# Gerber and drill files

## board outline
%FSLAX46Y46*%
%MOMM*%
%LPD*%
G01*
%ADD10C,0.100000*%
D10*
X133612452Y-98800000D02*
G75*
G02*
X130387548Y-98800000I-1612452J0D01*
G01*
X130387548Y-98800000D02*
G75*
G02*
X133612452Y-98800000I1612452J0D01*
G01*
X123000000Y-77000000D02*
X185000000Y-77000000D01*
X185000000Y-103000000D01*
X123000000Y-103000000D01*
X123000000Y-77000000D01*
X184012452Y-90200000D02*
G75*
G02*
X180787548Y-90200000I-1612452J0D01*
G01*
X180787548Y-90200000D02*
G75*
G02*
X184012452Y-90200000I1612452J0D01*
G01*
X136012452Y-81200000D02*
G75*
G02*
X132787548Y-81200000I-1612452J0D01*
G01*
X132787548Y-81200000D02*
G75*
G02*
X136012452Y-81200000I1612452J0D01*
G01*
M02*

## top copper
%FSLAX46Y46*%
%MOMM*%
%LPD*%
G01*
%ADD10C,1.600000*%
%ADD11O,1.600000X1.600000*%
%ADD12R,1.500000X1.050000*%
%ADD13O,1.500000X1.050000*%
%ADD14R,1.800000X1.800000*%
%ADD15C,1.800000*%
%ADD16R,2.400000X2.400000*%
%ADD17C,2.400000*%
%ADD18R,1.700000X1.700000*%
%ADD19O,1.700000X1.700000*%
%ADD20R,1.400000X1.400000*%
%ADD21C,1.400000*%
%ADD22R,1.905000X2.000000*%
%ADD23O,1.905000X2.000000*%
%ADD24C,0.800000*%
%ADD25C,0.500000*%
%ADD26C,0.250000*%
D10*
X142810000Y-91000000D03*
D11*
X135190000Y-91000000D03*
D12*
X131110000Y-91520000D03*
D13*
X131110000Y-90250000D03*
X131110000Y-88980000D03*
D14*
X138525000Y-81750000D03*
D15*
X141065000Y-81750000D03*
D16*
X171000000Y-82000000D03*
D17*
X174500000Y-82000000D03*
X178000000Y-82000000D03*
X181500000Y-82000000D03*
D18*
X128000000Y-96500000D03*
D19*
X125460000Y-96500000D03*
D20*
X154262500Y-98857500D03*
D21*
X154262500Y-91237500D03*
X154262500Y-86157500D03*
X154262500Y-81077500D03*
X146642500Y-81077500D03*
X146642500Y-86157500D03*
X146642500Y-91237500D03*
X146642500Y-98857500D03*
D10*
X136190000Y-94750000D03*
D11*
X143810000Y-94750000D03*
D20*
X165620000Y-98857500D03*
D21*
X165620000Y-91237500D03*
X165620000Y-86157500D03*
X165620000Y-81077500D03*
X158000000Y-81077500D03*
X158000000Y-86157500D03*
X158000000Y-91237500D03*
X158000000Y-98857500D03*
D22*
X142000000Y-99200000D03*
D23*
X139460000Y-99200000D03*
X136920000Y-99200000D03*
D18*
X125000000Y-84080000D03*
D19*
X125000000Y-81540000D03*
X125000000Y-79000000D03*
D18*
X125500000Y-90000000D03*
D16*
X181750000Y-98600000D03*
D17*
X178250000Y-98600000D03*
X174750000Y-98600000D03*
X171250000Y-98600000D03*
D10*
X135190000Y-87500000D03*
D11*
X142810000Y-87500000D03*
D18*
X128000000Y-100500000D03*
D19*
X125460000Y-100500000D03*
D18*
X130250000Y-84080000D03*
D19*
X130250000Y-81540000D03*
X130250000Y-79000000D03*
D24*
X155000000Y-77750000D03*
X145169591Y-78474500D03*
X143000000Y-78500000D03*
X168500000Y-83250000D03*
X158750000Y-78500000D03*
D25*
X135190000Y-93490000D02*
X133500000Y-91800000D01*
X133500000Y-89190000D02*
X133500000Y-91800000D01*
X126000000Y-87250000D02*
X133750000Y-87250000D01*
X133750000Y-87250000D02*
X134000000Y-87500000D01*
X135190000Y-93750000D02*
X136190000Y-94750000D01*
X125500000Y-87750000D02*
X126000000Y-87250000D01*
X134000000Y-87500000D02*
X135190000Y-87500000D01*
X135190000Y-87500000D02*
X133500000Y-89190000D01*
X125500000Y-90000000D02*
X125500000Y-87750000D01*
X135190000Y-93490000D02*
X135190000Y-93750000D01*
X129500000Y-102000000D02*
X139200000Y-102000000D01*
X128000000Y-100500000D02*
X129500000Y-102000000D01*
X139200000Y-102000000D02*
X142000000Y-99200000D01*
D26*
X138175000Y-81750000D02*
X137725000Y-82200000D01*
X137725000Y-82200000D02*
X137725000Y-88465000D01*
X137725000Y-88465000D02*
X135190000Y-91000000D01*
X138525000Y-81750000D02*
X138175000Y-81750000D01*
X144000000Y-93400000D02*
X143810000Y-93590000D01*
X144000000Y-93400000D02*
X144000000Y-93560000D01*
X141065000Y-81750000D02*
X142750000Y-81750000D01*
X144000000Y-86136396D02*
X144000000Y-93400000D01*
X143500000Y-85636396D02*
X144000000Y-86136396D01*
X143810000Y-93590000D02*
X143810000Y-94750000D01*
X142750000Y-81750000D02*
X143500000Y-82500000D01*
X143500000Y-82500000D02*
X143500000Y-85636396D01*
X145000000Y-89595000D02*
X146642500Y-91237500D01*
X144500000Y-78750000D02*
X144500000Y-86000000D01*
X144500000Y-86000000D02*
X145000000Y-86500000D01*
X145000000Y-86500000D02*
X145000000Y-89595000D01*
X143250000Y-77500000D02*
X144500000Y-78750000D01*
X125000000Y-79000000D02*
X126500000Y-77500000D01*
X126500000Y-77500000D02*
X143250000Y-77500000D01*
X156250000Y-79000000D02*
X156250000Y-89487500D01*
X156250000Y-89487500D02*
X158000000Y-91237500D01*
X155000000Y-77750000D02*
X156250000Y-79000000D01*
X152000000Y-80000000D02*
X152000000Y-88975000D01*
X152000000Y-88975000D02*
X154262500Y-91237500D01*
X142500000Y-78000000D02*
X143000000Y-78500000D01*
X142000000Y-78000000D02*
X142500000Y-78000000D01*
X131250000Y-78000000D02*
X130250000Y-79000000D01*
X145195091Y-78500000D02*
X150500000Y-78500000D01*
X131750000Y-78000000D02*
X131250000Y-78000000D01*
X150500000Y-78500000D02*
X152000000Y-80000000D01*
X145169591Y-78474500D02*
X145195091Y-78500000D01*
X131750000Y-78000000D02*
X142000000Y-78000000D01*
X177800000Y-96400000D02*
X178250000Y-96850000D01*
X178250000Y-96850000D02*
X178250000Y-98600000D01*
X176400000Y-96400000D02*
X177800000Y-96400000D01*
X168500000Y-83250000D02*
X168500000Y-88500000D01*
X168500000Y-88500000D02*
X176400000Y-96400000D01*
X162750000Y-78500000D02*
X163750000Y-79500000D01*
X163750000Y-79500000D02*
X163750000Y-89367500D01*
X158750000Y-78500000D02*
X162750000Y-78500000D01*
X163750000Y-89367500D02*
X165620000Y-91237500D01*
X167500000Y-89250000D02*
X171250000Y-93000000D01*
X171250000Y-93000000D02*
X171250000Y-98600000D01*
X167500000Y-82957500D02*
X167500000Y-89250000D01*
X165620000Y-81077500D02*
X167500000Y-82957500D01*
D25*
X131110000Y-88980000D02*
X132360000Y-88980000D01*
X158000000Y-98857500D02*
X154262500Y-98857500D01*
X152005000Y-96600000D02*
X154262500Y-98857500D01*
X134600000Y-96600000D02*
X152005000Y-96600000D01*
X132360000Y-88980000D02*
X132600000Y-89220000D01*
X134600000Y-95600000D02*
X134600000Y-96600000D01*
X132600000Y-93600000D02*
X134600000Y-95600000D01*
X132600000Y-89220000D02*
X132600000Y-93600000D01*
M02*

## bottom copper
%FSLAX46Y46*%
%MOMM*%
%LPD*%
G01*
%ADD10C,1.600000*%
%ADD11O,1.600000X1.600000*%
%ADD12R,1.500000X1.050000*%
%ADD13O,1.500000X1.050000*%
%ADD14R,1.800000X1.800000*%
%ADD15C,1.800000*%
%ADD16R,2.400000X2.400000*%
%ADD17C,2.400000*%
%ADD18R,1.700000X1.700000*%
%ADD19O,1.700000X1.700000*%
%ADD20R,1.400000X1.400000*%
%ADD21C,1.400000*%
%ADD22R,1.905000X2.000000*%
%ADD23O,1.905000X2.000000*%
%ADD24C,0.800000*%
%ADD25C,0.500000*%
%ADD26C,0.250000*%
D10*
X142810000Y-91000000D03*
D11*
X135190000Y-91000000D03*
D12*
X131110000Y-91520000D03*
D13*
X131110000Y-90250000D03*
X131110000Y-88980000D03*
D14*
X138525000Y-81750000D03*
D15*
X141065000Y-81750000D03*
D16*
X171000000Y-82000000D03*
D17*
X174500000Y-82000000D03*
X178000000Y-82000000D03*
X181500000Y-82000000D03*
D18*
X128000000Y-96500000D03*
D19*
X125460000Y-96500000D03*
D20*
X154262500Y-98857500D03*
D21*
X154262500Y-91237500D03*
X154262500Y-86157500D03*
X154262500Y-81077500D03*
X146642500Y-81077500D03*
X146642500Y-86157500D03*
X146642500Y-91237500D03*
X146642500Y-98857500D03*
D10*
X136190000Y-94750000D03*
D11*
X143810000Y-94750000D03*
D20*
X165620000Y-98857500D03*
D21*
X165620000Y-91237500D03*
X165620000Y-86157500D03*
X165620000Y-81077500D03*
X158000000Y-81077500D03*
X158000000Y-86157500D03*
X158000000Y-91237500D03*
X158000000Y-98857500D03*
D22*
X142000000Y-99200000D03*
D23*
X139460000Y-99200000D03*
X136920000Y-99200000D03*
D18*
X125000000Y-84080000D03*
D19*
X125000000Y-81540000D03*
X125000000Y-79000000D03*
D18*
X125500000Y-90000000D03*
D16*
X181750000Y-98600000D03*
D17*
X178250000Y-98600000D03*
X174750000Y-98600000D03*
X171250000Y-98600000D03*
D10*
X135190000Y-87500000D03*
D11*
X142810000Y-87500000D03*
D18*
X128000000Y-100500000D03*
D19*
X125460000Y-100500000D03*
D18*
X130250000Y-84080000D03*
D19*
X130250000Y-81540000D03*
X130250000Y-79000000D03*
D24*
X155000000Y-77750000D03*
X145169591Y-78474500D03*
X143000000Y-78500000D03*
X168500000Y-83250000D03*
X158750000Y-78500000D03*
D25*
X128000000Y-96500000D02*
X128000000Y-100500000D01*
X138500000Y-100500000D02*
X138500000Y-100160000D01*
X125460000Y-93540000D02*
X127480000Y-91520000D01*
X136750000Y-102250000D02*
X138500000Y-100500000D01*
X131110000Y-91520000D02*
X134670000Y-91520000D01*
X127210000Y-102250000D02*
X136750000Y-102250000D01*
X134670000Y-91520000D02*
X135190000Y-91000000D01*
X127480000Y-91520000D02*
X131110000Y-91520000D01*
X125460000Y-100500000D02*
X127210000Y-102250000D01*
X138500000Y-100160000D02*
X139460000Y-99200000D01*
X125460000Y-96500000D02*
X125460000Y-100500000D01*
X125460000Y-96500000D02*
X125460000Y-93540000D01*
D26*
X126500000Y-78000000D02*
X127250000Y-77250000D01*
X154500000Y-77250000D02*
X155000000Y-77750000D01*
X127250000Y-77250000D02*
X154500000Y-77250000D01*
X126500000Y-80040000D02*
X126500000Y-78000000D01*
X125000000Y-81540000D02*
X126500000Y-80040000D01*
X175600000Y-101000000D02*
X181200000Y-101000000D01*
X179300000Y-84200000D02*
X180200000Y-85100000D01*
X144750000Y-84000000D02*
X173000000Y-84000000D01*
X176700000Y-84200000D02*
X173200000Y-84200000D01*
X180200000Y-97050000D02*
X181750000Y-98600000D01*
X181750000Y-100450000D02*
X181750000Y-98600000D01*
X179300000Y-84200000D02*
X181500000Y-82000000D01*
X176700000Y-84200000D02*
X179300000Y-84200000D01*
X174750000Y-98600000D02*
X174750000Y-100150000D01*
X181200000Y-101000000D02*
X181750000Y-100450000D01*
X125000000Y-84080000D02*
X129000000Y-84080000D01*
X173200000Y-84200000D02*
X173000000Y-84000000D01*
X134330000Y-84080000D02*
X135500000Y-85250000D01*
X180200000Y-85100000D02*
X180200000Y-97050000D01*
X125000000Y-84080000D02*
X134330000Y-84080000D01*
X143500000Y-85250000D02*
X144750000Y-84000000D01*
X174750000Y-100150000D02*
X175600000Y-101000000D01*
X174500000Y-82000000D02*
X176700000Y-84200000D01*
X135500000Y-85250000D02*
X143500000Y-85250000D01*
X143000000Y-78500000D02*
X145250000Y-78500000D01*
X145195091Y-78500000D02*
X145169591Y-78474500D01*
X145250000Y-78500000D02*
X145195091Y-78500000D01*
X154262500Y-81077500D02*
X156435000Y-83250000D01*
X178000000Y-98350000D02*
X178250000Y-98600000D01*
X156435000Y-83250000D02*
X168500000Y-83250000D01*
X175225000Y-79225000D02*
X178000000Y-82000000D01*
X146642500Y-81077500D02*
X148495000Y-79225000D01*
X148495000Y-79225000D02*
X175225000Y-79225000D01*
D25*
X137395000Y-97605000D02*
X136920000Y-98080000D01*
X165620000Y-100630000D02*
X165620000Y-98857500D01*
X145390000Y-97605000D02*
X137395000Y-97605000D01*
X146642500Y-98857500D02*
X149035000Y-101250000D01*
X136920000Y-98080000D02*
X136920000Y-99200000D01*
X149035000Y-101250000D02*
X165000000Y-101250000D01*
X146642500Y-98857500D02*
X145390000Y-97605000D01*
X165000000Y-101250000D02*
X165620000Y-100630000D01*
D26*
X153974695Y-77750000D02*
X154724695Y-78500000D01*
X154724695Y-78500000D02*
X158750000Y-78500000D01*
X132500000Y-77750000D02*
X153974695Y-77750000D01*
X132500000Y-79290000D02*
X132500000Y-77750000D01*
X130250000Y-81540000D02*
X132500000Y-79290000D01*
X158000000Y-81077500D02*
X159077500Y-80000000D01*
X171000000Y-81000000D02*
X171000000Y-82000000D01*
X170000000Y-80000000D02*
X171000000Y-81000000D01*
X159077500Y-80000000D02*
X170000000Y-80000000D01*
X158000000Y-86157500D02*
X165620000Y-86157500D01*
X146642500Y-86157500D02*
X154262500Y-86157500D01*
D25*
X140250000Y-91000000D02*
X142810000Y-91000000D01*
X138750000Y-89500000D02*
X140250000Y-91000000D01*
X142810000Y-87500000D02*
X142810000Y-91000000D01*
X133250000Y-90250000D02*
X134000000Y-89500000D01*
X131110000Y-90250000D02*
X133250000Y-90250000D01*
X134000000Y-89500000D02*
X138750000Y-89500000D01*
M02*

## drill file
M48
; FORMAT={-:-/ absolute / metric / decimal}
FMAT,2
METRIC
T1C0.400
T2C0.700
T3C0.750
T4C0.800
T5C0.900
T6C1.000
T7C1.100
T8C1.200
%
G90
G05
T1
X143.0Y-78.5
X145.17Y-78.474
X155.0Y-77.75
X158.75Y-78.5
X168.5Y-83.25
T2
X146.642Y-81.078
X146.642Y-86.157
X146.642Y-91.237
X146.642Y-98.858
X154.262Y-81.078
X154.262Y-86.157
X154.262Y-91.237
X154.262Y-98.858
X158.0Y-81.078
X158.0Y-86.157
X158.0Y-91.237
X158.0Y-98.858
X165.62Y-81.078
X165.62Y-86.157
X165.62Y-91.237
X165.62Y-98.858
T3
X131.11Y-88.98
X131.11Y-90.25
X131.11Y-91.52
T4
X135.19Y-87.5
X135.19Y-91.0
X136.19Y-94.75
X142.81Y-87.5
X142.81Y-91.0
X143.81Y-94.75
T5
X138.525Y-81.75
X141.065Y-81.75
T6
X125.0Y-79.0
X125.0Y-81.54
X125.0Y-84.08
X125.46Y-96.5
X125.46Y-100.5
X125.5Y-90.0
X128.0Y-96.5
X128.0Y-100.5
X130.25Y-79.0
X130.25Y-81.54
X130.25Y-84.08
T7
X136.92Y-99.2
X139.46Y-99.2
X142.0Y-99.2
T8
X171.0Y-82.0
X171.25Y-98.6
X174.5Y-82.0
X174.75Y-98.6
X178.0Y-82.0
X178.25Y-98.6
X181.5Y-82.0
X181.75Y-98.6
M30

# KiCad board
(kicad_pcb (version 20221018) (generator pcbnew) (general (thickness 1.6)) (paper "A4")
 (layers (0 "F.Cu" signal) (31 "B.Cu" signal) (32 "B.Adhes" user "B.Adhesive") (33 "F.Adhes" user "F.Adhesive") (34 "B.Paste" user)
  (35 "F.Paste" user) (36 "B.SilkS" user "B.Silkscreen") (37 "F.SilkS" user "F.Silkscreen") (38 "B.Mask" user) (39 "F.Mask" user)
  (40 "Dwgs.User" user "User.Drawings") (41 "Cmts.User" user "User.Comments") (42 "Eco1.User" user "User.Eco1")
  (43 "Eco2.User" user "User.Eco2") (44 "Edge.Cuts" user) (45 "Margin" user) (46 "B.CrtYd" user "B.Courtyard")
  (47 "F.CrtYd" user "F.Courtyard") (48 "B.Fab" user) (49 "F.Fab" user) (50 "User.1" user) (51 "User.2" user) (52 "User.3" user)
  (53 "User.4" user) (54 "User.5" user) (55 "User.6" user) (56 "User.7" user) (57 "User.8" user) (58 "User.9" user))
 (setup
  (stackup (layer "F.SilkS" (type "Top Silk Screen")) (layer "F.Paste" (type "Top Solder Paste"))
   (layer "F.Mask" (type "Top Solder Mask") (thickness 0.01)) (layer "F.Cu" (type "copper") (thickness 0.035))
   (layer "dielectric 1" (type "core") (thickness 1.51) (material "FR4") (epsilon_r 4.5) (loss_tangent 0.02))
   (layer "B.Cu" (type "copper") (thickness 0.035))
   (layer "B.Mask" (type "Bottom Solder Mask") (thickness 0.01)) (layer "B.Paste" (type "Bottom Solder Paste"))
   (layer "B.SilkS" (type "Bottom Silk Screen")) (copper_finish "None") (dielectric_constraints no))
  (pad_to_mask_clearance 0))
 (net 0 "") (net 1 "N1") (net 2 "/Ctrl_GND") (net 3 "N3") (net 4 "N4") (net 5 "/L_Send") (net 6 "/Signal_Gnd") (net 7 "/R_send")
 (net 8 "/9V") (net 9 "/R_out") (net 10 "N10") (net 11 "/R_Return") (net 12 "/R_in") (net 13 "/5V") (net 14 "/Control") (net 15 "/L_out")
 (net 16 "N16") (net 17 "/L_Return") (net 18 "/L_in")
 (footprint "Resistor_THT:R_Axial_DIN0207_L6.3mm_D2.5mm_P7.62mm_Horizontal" (layer "F.Cu") (at 142.81 91 180)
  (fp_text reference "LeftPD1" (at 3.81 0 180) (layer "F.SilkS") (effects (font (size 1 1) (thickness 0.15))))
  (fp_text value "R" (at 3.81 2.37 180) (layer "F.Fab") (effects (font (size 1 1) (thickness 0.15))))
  (pad "1" thru_hole circle (at 0 0 180) (size 1.6 1.6) (drill 0.8) (layers "*.Cu" "*.Mask") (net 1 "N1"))
  (pad "2" thru_hole oval (at 7.62 0 180) (size 1.6 1.6) (drill 0.8) (layers "*.Cu" "*.Mask") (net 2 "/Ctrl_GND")))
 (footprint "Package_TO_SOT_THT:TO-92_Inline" (layer "F.Cu") (at 131.11 91.52 90)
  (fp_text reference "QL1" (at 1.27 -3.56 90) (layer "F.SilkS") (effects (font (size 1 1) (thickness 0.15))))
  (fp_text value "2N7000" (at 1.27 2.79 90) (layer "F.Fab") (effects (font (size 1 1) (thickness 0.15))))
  (pad "1" thru_hole rect (at 0 0 90) (size 1.05 1.5) (drill 0.75) (layers "*.Cu" "*.Mask") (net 2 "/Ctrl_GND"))
  (pad "2" thru_hole oval (at 1.27 0 90) (size 1.05 1.5) (drill 0.75) (layers "*.Cu" "*.Mask") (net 1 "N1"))
  (pad "3" thru_hole oval (at 2.54 0 90) (size 1.05 1.5) (drill 0.75) (layers "*.Cu" "*.Mask") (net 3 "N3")))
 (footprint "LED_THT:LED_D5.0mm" (layer "F.Cu") (at 138.525 81.75)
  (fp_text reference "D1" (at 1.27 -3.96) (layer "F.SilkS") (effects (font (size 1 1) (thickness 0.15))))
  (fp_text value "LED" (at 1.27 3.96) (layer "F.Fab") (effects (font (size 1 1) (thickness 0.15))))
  (pad "1" thru_hole rect (at 0 0) (size 1.8 1.8) (drill 0.9) (layers "*.Cu" "*.Mask") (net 2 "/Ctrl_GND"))
  (pad "2" thru_hole circle (at 2.54 0) (size 1.8 1.8) (drill 0.9) (layers "*.Cu" "*.Mask") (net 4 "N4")))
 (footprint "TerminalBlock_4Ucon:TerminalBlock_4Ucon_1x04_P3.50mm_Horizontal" (layer "F.Cu") (at 171 82)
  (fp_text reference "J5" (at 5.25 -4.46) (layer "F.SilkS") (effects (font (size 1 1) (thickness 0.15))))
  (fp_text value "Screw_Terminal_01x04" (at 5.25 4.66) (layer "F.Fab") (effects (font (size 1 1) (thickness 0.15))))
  (pad "1" thru_hole rect (at 0 0) (size 2.4 2.4) (drill 1.2) (layers "*.Cu" "*.Mask") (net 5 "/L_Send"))
  (pad "2" thru_hole circle (at 3.5 0) (size 2.4 2.4) (drill 1.2) (layers "*.Cu" "*.Mask") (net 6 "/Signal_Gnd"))
  (pad "3" thru_hole circle (at 7 0) (size 2.4 2.4) (drill 1.2) (layers "*.Cu" "*.Mask") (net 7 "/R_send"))
  (pad "4" thru_hole circle (at 10.5 0) (size 2.4 2.4) (drill 1.2) (layers "*.Cu" "*.Mask") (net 6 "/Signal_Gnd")))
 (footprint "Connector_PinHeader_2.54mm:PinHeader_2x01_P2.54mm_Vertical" (layer "F.Cu") (at 128 96.5 180)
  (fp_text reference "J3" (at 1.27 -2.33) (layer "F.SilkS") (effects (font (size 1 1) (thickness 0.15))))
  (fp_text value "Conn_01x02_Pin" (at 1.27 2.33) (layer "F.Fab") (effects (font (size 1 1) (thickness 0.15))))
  (pad "1" thru_hole rect (at 0 0 180) (size 1.7 1.7) (drill 1) (layers "*.Cu" "*.Mask") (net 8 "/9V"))
  (pad "2" thru_hole oval (at 2.54 0 180) (size 1.7 1.7) (drill 1) (layers "*.Cu" "*.Mask") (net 2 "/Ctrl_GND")))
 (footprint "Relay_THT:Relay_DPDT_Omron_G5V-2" (layer "F.Cu") (at 154.2625 98.8575 180)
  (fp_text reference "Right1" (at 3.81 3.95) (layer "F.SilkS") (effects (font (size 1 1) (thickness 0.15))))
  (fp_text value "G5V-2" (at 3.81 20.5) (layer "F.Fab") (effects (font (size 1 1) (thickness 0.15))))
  (pad "1" thru_hole rect (at 0 0 180) (size 1.4 1.4) (drill 0.7) (layers "*.Cu" "*.Mask") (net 3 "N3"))
  (pad "4" thru_hole circle (at 0 7.62 180) (size 1.4 1.4) (drill 0.7) (layers "*.Cu" "*.Mask") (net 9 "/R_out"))
  (pad "6" thru_hole circle (at 0 12.7 180) (size 1.4 1.4) (drill 0.7) (layers "*.Cu" "*.Mask") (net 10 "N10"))
  (pad "8" thru_hole circle (at 0 17.78 180) (size 1.4 1.4) (drill 0.7) (layers "*.Cu" "*.Mask") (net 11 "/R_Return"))
  (pad "9" thru_hole circle (at 7.62 17.78 180) (size 1.4 1.4) (drill 0.7) (layers "*.Cu" "*.Mask") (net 7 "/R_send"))
  (pad "11" thru_hole circle (at 7.62 12.7 180) (size 1.4 1.4) (drill 0.7) (layers "*.Cu" "*.Mask") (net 10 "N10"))
  (pad "13" thru_hole circle (at 7.62 7.62 180) (size 1.4 1.4) (drill 0.7) (layers "*.Cu" "*.Mask") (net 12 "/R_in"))
  (pad "16" thru_hole circle (at 7.62 0 180) (size 1.4 1.4) (drill 0.7) (layers "*.Cu" "*.Mask") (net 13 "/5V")))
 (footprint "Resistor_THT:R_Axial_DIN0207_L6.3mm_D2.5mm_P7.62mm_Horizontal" (layer "F.Cu") (at 136.19 94.75)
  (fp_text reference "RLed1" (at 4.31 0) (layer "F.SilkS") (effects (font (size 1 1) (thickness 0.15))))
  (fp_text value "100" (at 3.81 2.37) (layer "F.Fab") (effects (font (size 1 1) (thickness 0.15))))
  (pad "1" thru_hole circle (at 0 0) (size 1.6 1.6) (drill 0.8) (layers "*.Cu" "*.Mask") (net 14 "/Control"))
  (pad "2" thru_hole oval (at 7.62 0) (size 1.6 1.6) (drill 0.8) (layers "*.Cu" "*.Mask") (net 4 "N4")))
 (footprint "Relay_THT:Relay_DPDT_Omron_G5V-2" (layer "F.Cu") (at 165.62 98.8575 180)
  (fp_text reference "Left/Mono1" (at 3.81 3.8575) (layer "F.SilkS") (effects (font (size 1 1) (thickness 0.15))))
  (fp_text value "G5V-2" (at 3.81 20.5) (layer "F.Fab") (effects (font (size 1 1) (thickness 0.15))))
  (pad "1" thru_hole rect (at 0 0 180) (size 1.4 1.4) (drill 0.7) (layers "*.Cu" "*.Mask") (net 13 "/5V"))
  (pad "4" thru_hole circle (at 0 7.62 180) (size 1.4 1.4) (drill 0.7) (layers "*.Cu" "*.Mask") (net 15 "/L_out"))
  (pad "6" thru_hole circle (at 0 12.7 180) (size 1.4 1.4) (drill 0.7) (layers "*.Cu" "*.Mask") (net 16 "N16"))
  (pad "8" thru_hole circle (at 0 17.78 180) (size 1.4 1.4) (drill 0.7) (layers "*.Cu" "*.Mask") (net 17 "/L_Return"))
  (pad "9" thru_hole circle (at 7.62 17.78 180) (size 1.4 1.4) (drill 0.7) (layers "*.Cu" "*.Mask") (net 5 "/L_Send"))
  (pad "11" thru_hole circle (at 7.62 12.7 180) (size 1.4 1.4) (drill 0.7) (layers "*.Cu" "*.Mask") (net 16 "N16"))
  (pad "13" thru_hole circle (at 7.62 7.62 180) (size 1.4 1.4) (drill 0.7) (layers "*.Cu" "*.Mask") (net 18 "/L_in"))
  (pad "16" thru_hole circle (at 7.62 0 180) (size 1.4 1.4) (drill 0.7) (layers "*.Cu" "*.Mask") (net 3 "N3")))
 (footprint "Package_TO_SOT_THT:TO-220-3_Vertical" (layer "F.Cu") (at 142 99.2 180)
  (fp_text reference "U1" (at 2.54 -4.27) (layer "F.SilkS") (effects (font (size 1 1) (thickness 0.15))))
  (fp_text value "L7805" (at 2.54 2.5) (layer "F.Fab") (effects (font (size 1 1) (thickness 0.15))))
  (pad "1" thru_hole rect (at 0 0 180) (size 1.905 2) (drill 1.1) (layers "*.Cu" "*.Mask") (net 8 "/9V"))
  (pad "2" thru_hole oval (at 2.54 0 180) (size 1.905 2) (drill 1.1) (layers "*.Cu" "*.Mask") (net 2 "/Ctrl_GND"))
  (pad "3" thru_hole oval (at 5.08 0 180) (size 1.905 2) (drill 1.1) (layers "*.Cu" "*.Mask") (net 13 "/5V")))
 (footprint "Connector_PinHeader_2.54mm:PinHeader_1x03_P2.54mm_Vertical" (layer "F.Cu") (at 125 84.08 180)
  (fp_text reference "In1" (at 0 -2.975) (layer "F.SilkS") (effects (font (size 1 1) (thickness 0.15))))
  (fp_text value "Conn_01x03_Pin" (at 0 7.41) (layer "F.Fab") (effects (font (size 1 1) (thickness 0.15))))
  (pad "1" thru_hole rect (at 0 0 180) (size 1.7 1.7) (drill 1) (layers "*.Cu" "*.Mask") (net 6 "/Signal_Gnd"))
  (pad "2" thru_hole oval (at 0 2.54 180) (size 1.7 1.7) (drill 1) (layers "*.Cu" "*.Mask") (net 18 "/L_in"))
  (pad "3" thru_hole oval (at 0 5.08 180) (size 1.7 1.7) (drill 1) (layers "*.Cu" "*.Mask") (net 12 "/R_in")))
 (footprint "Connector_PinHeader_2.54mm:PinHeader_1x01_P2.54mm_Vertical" (layer "F.Cu") (at 125.5 90 90)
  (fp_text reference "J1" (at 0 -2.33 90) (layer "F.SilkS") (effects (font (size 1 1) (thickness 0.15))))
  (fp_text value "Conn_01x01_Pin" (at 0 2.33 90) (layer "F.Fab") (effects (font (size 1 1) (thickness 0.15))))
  (pad "1" thru_hole rect (at 0 0 90) (size 1.7 1.7) (drill 1) (layers "*.Cu" "*.Mask") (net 14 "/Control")))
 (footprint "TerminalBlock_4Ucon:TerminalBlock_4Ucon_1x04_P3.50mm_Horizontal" (layer "F.Cu") (at 181.75 98.6 180)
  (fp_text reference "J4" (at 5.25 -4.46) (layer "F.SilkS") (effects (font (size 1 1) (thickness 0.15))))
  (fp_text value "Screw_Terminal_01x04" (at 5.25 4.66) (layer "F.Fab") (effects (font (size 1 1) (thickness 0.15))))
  (pad "1" thru_hole rect (at 0 0 180) (size 2.4 2.4) (drill 1.2) (layers "*.Cu" "*.Mask") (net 6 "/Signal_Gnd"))
  (pad "2" thru_hole circle (at 3.5 0 180) (size 2.4 2.4) (drill 1.2) (layers "*.Cu" "*.Mask") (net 11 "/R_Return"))
  (pad "3" thru_hole circle (at 7 0 180) (size 2.4 2.4) (drill 1.2) (layers "*.Cu" "*.Mask") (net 6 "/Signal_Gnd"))
  (pad "4" thru_hole circle (at 10.5 0 180) (size 2.4 2.4) (drill 1.2) (layers "*.Cu" "*.Mask") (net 17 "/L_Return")))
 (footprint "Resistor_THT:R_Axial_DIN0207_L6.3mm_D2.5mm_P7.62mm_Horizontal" (layer "F.Cu") (at 135.19 87.5)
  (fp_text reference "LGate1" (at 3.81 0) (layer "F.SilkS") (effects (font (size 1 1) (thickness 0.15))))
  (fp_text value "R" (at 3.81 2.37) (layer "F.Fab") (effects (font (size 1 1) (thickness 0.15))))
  (pad "1" thru_hole circle (at 0 0) (size 1.6 1.6) (drill 0.8) (layers "*.Cu" "*.Mask") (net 14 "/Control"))
  (pad "2" thru_hole oval (at 7.62 0) (size 1.6 1.6) (drill 0.8) (layers "*.Cu" "*.Mask") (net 1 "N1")))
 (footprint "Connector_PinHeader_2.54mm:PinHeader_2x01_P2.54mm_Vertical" (layer "F.Cu") (at 128 100.5 180)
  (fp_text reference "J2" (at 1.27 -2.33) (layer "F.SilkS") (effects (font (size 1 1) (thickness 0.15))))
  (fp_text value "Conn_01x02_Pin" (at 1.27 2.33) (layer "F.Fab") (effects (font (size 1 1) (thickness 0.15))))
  (pad "1" thru_hole rect (at 0 0 180) (size 1.7 1.7) (drill 1) (layers "*.Cu" "*.Mask") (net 8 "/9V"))
  (pad "2" thru_hole oval (at 2.54 0 180) (size 1.7 1.7) (drill 1) (layers "*.Cu" "*.Mask") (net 2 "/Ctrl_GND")))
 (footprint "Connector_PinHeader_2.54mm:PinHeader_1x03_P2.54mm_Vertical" (layer "F.Cu") (at 130.25 84.08 180)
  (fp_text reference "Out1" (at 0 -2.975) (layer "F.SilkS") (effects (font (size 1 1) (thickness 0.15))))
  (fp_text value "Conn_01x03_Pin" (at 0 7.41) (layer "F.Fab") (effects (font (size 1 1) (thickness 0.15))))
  (pad "1" thru_hole rect (at 0 0 180) (size 1.7 1.7) (drill 1) (layers "*.Cu" "*.Mask") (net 6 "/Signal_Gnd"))
  (pad "2" thru_hole oval (at 0 2.54 180) (size 1.7 1.7) (drill 1) (layers "*.Cu" "*.Mask") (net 15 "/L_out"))
  (pad "3" thru_hole oval (at 0 5.08 180) (size 1.7 1.7) (drill 1) (layers "*.Cu" "*.Mask") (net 9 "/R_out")))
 (gr_circle (center 132 98.8) (end 131.8 97.2) (stroke (width 0.1) (type default)) (fill none) (layer "Edge.Cuts"))
 (gr_rect (start 123 77) (end 185 103) (stroke (width 0.1) (type default)) (fill none) (layer "Edge.Cuts"))
 (gr_circle (center 182.4 90.2) (end 182.2 88.6) (stroke (width 0.1) (type default)) (fill none) (layer "Edge.Cuts"))
 (gr_circle (center 134.4 81.2) (end 134.2 79.6) (stroke (width 0.1) (type default)) (fill none) (layer "Edge.Cuts"))
 (segment (start 135.19 93.49) (end 133.5 91.8) (width 0.5) (layer "F.Cu") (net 14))
 (segment (start 133.5 89.19) (end 133.5 91.8) (width 0.5) (layer "F.Cu") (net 14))
 (segment (start 126 87.25) (end 133.75 87.25) (width 0.5) (layer "F.Cu") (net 14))
 (segment (start 133.75 87.25) (end 134 87.5) (width 0.5) (layer "F.Cu") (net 14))
 (segment (start 135.19 93.75) (end 136.19 94.75) (width 0.5) (layer "F.Cu") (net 14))
 (segment (start 125.5 87.75) (end 126 87.25) (width 0.5) (layer "F.Cu") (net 14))
 (segment (start 134 87.5) (end 135.19 87.5) (width 0.5) (layer "F.Cu") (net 14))
 (segment (start 135.19 87.5) (end 133.5 89.19) (width 0.5) (layer "F.Cu") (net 14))
 (segment (start 125.5 90) (end 125.5 87.75) (width 0.5) (layer "F.Cu") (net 14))
 (segment (start 135.19 93.49) (end 135.19 93.75) (width 0.5) (layer "F.Cu") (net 14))
 (segment (start 129.5 102) (end 139.2 102) (width 0.5) (layer "F.Cu") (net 8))
 (segment (start 128 100.5) (end 129.5 102) (width 0.5) (layer "F.Cu") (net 8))
 (segment (start 139.2 102) (end 142 99.2) (width 0.5) (layer "F.Cu") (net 8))
 (segment (start 128 96.5) (end 128 100.5) (width 0.5) (layer "B.Cu") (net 8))
 (segment (start 138.175 81.75) (end 137.725 82.2) (width 0.25) (layer "F.Cu") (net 2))
 (segment (start 137.725 82.2) (end 137.725 88.465) (width 0.25) (layer "F.Cu") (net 2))
 (segment (start 137.725 88.465) (end 135.19 91) (width 0.25) (layer "F.Cu") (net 2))
 (segment (start 138.525 81.75) (end 138.175 81.75) (width 0.25) (layer "F.Cu") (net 2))
 (segment (start 138.5 100.5) (end 138.5 100.16) (width 0.5) (layer "B.Cu") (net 2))
 (segment (start 125.46 93.54) (end 127.48 91.52) (width 0.5) (layer "B.Cu") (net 2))
 (segment (start 136.75 102.25) (end 138.5 100.5) (width 0.5) (layer "B.Cu") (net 2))
 (segment (start 131.11 91.52) (end 134.67 91.52) (width 0.5) (layer "B.Cu") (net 2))
 (segment (start 127.21 102.25) (end 136.75 102.25) (width 0.5) (layer "B.Cu") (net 2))
 (segment (start 134.67 91.52) (end 135.19 91) (width 0.5) (layer "B.Cu") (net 2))
 (segment (start 127.48 91.52) (end 131.11 91.52) (width 0.5) (layer "B.Cu") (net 2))
 (segment (start 125.46 100.5) (end 127.21 102.25) (width 0.5) (layer "B.Cu") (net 2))
 (segment (start 138.5 100.16) (end 139.46 99.2) (width 0.5) (layer "B.Cu") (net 2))
 (segment (start 125.46 96.5) (end 125.46 100.5) (width 0.5) (layer "B.Cu") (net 2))
 (segment (start 125.46 96.5) (end 125.46 93.54) (width 0.5) (layer "B.Cu") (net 2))
 (segment (start 144 93.4) (end 143.81 93.59) (width 0.25) (layer "F.Cu") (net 4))
 (segment (start 144 93.4) (end 144 93.56) (width 0.25) (layer "F.Cu") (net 4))
 (segment (start 141.065 81.75) (end 142.75 81.75) (width 0.25) (layer "F.Cu") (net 4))
 (segment (start 144 86.136396) (end 144 93.4) (width 0.25) (layer "F.Cu") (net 4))
 (segment (start 143.5 85.636396) (end 144 86.136396) (width 0.25) (layer "F.Cu") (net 4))
 (segment (start 143.81 93.59) (end 143.81 94.75) (width 0.25) (layer "F.Cu") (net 4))
 (segment (start 142.75 81.75) (end 143.5 82.5) (width 0.25) (layer "F.Cu") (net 4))
 (segment (start 143.5 82.5) (end 143.5 85.636396) (width 0.25) (layer "F.Cu") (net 4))
 (segment (start 145 89.595) (end 146.6425 91.2375) (width 0.25) (layer "F.Cu") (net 12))
 (segment (start 144.5 78.75) (end 144.5 86) (width 0.25) (layer "F.Cu") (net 12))
 (segment (start 144.5 86) (end 145 86.5) (width 0.25) (layer "F.Cu") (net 12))
 (segment (start 145 86.5) (end 145 89.595) (width 0.25) (layer "F.Cu") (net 12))
 (segment (start 143.25 77.5) (end 144.5 78.75) (width 0.25) (layer "F.Cu") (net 12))
 (segment (start 125 79) (end 126.5 77.5) (width 0.25) (layer "F.Cu") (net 12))
 (segment (start 126.5 77.5) (end 143.25 77.5) (width 0.25) (layer "F.Cu") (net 12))
 (segment (start 156.25 79) (end 156.25 89.4875) (width 0.25) (layer "F.Cu") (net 18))
 (segment (start 156.25 89.4875) (end 158 91.2375) (width 0.25) (layer "F.Cu") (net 18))
 (segment (start 155 77.75) (end 156.25 79) (width 0.25) (layer "F.Cu") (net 18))
 (via (at 155 77.75) (size 0.8) (drill 0.4) (layers "F.Cu" "B.Cu") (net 18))
 (segment (start 126.5 78) (end 127.25 77.25) (width 0.25) (layer "B.Cu") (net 18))
 (segment (start 154.5 77.25) (end 155 77.75) (width 0.25) (layer "B.Cu") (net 18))
 (segment (start 127.25 77.25) (end 154.5 77.25) (width 0.25) (layer "B.Cu") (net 18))
 (segment (start 126.5 80.04) (end 126.5 78) (width 0.25) (layer "B.Cu") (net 18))
 (segment (start 125 81.54) (end 126.5 80.04) (width 0.25) (layer "B.Cu") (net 18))
 (segment (start 175.6 101) (end 181.2 101) (width 0.25) (layer "B.Cu") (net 6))
 (segment (start 179.3 84.2) (end 180.2 85.1) (width 0.25) (layer "B.Cu") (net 6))
 (segment (start 144.75 84) (end 173 84) (width 0.25) (layer "B.Cu") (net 6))
 (segment (start 176.7 84.2) (end 173.2 84.2) (width 0.25) (layer "B.Cu") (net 6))
 (segment (start 180.2 97.05) (end 181.75 98.6) (width 0.25) (layer "B.Cu") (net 6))
 (segment (start 181.75 100.45) (end 181.75 98.6) (width 0.25) (layer "B.Cu") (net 6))
 (segment (start 179.3 84.2) (end 181.5 82) (width 0.25) (layer "B.Cu") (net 6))
 (segment (start 176.7 84.2) (end 179.3 84.2) (width 0.25) (layer "B.Cu") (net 6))
 (segment (start 174.75 98.6) (end 174.75 100.15) (width 0.25) (layer "B.Cu") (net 6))
 (segment (start 181.2 101) (end 181.75 100.45) (width 0.25) (layer "B.Cu") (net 6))
 (segment (start 125 84.08) (end 129 84.08) (width 0.25) (layer "B.Cu") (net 6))
 (segment (start 173.2 84.2) (end 173 84) (width 0.25) (layer "B.Cu") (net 6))
 (segment (start 134.33 84.08) (end 135.5 85.25) (width 0.25) (layer "B.Cu") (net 6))
 (segment (start 180.2 85.1) (end 180.2 97.05) (width 0.25) (layer "B.Cu") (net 6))
 (segment (start 125 84.08) (end 134.33 84.08) (width 0.25) (layer "B.Cu") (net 6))
 (segment (start 143.5 85.25) (end 144.75 84) (width 0.25) (layer "B.Cu") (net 6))
 (segment (start 174.75 100.15) (end 175.6 101) (width 0.25) (layer "B.Cu") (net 6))
 (segment (start 174.5 82) (end 176.7 84.2) (width 0.25) (layer "B.Cu") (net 6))
 (segment (start 135.5 85.25) (end 143.5 85.25) (width 0.25) (layer "B.Cu") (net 6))
 (segment (start 152 80) (end 152 88.975) (width 0.25) (layer "F.Cu") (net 9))
 (segment (start 152 88.975) (end 154.2625 91.2375) (width 0.25) (layer "F.Cu") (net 9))
 (segment (start 142.5 78) (end 143 78.5) (width 0.25) (layer "F.Cu") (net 9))
 (segment (start 142 78) (end 142.5 78) (width 0.25) (layer "F.Cu") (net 9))
 (segment (start 131.25 78) (end 130.25 79) (width 0.25) (layer "F.Cu") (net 9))
 (segment (start 145.195091 78.5) (end 150.5 78.5) (width 0.25) (layer "F.Cu") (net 9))
 (segment (start 131.75 78) (end 131.25 78) (width 0.25) (layer "F.Cu") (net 9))
 (segment (start 150.5 78.5) (end 152 80) (width 0.25) (layer "F.Cu") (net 9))
 (segment (start 145.169591 78.4745) (end 145.195091 78.5) (width 0.25) (layer "F.Cu") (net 9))
 (segment (start 131.75 78) (end 142 78) (width 0.25) (layer "F.Cu") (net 9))
 (via (at 145.169591 78.4745) (size 0.8) (drill 0.4) (layers "F.Cu" "B.Cu") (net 9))
 (via (at 143 78.5) (size 0.8) (drill 0.4) (layers "F.Cu" "B.Cu") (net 9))
 (segment (start 143 78.5) (end 145.25 78.5) (width 0.25) (layer "B.Cu") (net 9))
 (segment (start 145.195091 78.5) (end 145.169591 78.4745) (width 0.25) (layer "B.Cu") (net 9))
 (segment (start 145.25 78.5) (end 145.195091 78.5) (width 0.25) (layer "B.Cu") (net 9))
 (segment (start 177.8 96.4) (end 178.25 96.85) (width 0.25) (layer "F.Cu") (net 11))
 (segment (start 178.25 96.85) (end 178.25 98.6) (width 0.25) (layer "F.Cu") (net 11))
 (segment (start 176.4 96.4) (end 177.8 96.4) (width 0.25) (layer "F.Cu") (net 11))
 (segment (start 168.5 83.25) (end 168.5 88.5) (width 0.25) (layer "F.Cu") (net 11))
 (segment (start 168.5 88.5) (end 176.4 96.4) (width 0.25) (layer "F.Cu") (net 11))
 (via (at 168.5 83.25) (size 0.8) (drill 0.4) (layers "F.Cu" "B.Cu") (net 11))
 (segment (start 154.2625 81.0775) (end 156.435 83.25) (width 0.25) (layer "B.Cu") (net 11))
 (segment (start 178 98.35) (end 178.25 98.6) (width 0.25) (layer "B.Cu") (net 11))
 (segment (start 156.435 83.25) (end 168.5 83.25) (width 0.25) (layer "B.Cu") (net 11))
 (segment (start 175.225 79.225) (end 178 82) (width 0.25) (layer "B.Cu") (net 7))
 (segment (start 146.6425 81.0775) (end 148.495 79.225) (width 0.25) (layer "B.Cu") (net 7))
 (segment (start 148.495 79.225) (end 175.225 79.225) (width 0.25) (layer "B.Cu") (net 7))
 (segment (start 137.395 97.605) (end 136.92 98.08) (width 0.5) (layer "B.Cu") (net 13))
 (segment (start 165.62 100.63) (end 165.62 98.8575) (width 0.5) (layer "B.Cu") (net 13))
 (segment (start 145.39 97.605) (end 137.395 97.605) (width 0.5) (layer "B.Cu") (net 13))
 (segment (start 146.6425 98.8575) (end 149.035 101.25) (width 0.5) (layer "B.Cu") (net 13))
 (segment (start 136.92 98.08) (end 136.92 99.2) (width 0.5) (layer "B.Cu") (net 13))
 (segment (start 149.035 101.25) (end 165 101.25) (width 0.5) (layer "B.Cu") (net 13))
 (segment (start 146.6425 98.8575) (end 145.39 97.605) (width 0.5) (layer "B.Cu") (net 13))
 (segment (start 165 101.25) (end 165.62 100.63) (width 0.5) (layer "B.Cu") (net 13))
 (segment (start 162.75 78.5) (end 163.75 79.5) (width 0.25) (layer "F.Cu") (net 15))
 (segment (start 163.75 79.5) (end 163.75 89.3675) (width 0.25) (layer "F.Cu") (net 15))
 (segment (start 158.75 78.5) (end 162.75 78.5) (width 0.25) (layer "F.Cu") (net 15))
 (segment (start 163.75 89.3675) (end 165.62 91.2375) (width 0.25) (layer "F.Cu") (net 15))
 (via (at 158.75 78.5) (size 0.8) (drill 0.4) (layers "F.Cu" "B.Cu") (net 15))
 (segment (start 153.974695 77.75) (end 154.724695 78.5) (width 0.25) (layer "B.Cu") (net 15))
 (segment (start 154.724695 78.5) (end 158.75 78.5) (width 0.25) (layer "B.Cu") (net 15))
 (segment (start 132.5 77.75) (end 153.974695 77.75) (width 0.25) (layer "B.Cu") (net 15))
 (segment (start 132.5 79.29) (end 132.5 77.75) (width 0.25) (layer "B.Cu") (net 15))
 (segment (start 130.25 81.54) (end 132.5 79.29) (width 0.25) (layer "B.Cu") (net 15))
 (segment (start 167.5 89.25) (end 171.25 93) (width 0.25) (layer "F.Cu") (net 17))
 (segment (start 171.25 93) (end 171.25 98.6) (width 0.25) (layer "F.Cu") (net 17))
 (segment (start 167.5 82.9575) (end 167.5 89.25) (width 0.25) (layer "F.Cu") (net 17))
 (segment (start 165.62 81.0775) (end 167.5 82.9575) (width 0.25) (layer "F.Cu") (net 17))
 (segment (start 158 81.0775) (end 159.0775 80) (width 0.25) (layer "B.Cu") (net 5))
 (segment (start 171 81) (end 171 82) (width 0.25) (layer "B.Cu") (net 5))
 (segment (start 170 80) (end 171 81) (width 0.25) (layer "B.Cu") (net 5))
 (segment (start 159.0775 80) (end 170 80) (width 0.25) (layer "B.Cu") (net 5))
 (segment (start 158 86.1575) (end 165.62 86.1575) (width 0.25) (layer "B.Cu") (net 16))
 (segment (start 146.6425 86.1575) (end 154.2625 86.1575) (width 0.25) (layer "B.Cu") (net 10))
 (segment (start 131.11 88.98) (end 132.36 88.98) (width 0.5) (layer "F.Cu") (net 3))
 (segment (start 158 98.8575) (end 154.2625 98.8575) (width 0.5) (layer "F.Cu") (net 3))
 (segment (start 152.005 96.6) (end 154.2625 98.8575) (width 0.5) (layer "F.Cu") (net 3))
 (segment (start 134.6 96.6) (end 152.005 96.6) (width 0.5) (layer "F.Cu") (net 3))
 (segment (start 132.36 88.98) (end 132.6 89.22) (width 0.5) (layer "F.Cu") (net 3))
 (segment (start 134.6 95.6) (end 134.6 96.6) (width 0.5) (layer "F.Cu") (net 3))
 (segment (start 132.6 93.6) (end 134.6 95.6) (width 0.5) (layer "F.Cu") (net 3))
 (segment (start 132.6 89.22) (end 132.6 93.6) (width 0.5) (layer "F.Cu") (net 3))
 (segment (start 140.25 91) (end 142.81 91) (width 0.5) (layer "B.Cu") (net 1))
 (segment (start 138.75 89.5) (end 140.25 91) (width 0.5) (layer "B.Cu") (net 1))
 (segment (start 142.81 87.5) (end 142.81 91) (width 0.5) (layer "B.Cu") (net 1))
 (segment (start 133.25 90.25) (end 134 89.5) (width 0.5) (layer "B.Cu") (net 1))
 (segment (start 131.11 90.25) (end 133.25 90.25) (width 0.5) (layer "B.Cu") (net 1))
 (segment (start 134 89.5) (end 138.75 89.5) (width 0.5) (layer "B.Cu") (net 1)))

